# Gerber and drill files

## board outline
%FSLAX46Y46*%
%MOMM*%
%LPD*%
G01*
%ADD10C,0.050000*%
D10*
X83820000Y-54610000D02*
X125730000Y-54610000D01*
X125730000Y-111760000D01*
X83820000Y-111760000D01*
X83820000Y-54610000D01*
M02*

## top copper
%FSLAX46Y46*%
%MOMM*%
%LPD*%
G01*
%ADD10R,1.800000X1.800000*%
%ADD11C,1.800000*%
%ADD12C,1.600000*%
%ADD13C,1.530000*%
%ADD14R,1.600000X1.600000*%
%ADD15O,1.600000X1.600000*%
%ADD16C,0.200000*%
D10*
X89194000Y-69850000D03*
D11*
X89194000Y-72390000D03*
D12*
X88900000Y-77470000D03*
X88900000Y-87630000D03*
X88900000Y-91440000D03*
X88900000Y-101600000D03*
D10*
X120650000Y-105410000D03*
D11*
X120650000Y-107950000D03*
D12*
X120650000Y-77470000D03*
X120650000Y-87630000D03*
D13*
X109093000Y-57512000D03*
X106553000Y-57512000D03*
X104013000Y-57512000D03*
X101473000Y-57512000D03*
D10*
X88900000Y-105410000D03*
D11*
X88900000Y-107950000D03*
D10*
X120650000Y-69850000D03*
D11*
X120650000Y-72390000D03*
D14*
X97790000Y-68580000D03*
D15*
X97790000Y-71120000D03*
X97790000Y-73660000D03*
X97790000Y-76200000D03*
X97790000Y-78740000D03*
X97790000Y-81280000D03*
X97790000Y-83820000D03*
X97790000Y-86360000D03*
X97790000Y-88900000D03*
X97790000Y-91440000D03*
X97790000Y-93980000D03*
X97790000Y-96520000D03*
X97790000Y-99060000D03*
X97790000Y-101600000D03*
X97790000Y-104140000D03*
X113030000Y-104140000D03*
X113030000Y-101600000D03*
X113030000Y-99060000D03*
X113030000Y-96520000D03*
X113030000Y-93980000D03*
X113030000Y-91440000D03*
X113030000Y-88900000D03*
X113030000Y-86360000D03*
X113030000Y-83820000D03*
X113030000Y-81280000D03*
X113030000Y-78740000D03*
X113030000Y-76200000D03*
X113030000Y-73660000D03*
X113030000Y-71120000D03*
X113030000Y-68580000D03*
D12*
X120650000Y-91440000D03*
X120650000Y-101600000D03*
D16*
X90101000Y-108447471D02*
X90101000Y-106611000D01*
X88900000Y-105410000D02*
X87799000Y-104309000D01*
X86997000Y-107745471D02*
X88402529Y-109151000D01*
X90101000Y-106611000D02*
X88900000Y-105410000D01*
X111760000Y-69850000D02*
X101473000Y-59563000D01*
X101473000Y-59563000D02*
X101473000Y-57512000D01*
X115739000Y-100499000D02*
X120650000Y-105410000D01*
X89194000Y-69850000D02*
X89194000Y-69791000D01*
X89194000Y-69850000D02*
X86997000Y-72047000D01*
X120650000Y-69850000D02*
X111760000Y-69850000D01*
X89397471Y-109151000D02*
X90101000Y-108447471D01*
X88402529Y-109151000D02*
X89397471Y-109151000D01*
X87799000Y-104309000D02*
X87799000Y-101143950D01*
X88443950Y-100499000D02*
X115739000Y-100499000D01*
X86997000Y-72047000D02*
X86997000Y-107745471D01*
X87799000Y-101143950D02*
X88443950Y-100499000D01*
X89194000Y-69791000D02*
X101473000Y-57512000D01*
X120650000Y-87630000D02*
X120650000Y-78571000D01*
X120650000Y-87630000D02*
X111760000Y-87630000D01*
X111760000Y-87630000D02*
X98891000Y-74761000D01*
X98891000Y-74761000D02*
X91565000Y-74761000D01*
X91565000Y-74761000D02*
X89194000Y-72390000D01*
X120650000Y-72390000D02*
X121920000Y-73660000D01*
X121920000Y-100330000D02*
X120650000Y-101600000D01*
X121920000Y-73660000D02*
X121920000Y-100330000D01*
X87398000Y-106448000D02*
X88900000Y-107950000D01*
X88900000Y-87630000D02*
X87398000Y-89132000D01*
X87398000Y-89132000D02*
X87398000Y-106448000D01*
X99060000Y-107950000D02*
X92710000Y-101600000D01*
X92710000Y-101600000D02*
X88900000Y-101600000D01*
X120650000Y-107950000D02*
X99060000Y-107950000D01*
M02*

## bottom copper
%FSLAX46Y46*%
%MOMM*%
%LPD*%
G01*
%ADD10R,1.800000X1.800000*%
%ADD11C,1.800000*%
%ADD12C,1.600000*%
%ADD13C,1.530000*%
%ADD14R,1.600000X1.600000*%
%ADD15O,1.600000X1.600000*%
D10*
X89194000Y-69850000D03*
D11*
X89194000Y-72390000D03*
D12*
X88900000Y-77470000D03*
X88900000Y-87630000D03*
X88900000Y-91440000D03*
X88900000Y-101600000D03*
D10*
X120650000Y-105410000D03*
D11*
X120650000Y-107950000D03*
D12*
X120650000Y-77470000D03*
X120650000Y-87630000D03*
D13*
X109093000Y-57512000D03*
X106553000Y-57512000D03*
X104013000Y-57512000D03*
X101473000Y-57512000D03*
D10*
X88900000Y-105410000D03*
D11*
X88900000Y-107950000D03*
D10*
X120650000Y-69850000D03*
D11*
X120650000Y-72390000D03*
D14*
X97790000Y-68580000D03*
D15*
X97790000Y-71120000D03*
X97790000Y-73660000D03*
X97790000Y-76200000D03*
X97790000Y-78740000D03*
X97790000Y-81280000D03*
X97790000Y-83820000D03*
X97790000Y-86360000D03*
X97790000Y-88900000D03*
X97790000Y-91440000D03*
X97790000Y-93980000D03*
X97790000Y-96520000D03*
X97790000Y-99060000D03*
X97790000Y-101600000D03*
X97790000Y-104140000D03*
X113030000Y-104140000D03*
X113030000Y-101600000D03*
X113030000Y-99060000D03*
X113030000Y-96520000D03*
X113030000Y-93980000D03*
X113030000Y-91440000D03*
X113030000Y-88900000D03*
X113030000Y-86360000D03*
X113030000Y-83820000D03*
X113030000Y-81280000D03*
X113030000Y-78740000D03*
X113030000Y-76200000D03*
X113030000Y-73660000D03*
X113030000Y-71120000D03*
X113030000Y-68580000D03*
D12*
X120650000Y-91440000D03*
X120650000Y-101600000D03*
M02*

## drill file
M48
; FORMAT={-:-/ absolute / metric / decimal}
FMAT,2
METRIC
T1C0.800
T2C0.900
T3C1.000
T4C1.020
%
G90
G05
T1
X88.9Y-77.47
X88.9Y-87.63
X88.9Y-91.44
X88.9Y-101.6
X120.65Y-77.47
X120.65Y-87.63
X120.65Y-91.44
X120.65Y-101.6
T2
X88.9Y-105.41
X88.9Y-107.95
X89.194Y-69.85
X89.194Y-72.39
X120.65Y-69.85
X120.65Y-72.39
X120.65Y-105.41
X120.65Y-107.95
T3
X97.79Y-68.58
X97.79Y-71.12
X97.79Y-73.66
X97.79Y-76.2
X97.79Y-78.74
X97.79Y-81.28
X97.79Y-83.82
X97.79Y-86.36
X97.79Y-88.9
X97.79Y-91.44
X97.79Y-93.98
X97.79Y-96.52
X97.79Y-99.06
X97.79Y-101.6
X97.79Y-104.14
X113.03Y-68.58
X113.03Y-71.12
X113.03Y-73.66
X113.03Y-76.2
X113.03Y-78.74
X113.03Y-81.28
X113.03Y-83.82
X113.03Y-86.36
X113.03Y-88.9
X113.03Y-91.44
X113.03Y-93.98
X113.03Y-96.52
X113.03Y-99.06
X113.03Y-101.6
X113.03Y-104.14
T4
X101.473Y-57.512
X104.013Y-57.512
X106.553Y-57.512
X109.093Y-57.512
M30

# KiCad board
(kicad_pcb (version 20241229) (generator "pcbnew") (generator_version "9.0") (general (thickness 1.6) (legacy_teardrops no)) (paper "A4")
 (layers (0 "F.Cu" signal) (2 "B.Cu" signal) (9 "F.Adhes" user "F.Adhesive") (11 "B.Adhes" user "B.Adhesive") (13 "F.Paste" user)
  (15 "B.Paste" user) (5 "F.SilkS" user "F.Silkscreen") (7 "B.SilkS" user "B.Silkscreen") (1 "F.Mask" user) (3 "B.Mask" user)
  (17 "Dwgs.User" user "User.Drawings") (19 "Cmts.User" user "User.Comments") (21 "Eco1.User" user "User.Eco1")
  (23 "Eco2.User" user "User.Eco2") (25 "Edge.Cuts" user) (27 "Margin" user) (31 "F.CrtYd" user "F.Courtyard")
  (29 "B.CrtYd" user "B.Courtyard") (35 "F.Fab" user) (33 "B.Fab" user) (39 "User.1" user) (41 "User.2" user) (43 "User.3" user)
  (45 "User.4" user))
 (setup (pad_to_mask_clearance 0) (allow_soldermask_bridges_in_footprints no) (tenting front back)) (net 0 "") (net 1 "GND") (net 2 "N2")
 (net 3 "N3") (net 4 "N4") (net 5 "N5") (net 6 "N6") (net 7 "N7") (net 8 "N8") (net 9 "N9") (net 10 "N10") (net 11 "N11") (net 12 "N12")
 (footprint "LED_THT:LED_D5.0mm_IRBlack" (layer "F.Cu") (at 89.194 69.85 -90)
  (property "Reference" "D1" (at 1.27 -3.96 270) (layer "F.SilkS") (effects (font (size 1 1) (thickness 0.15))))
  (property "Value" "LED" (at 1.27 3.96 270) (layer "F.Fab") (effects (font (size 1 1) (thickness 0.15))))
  (pad "1" thru_hole rect (at 0 0 270) (size 1.8 1.8) (drill 0.9) (layers "*.Cu" "*.Mask") (remove_unused_layers no) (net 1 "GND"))
  (pad "2" thru_hole circle (at 2.54 0 270) (size 1.8 1.8) (drill 0.9) (layers "*.Cu" "*.Mask") (remove_unused_layers no) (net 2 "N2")))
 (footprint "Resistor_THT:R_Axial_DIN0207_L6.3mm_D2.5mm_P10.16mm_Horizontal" (layer "F.Cu") (at 88.9 77.47 -90)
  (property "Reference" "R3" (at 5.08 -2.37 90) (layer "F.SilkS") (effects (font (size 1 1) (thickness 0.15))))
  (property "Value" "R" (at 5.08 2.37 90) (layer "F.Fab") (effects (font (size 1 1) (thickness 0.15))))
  (pad "1" thru_hole circle (at 0 0 270) (size 1.6 1.6) (drill 0.8) (layers "*.Cu" "*.Mask") (remove_unused_layers no) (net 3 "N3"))
  (pad "2" thru_hole circle (at 10.16 0 270) (size 1.6 1.6) (drill 0.8) (layers "*.Cu" "*.Mask") (remove_unused_layers no) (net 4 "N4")))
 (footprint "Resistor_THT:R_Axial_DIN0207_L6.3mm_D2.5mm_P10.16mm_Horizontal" (layer "F.Cu") (at 88.9 91.44 -90)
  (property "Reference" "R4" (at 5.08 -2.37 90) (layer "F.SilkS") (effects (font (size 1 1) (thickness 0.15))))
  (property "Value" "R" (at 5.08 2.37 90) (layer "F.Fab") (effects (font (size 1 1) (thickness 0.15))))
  (pad "1" thru_hole circle (at 0 0 270) (size 1.6 1.6) (drill 0.8) (layers "*.Cu" "*.Mask") (remove_unused_layers no) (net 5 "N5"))
  (pad "2" thru_hole circle (at 10.16 0 270) (size 1.6 1.6) (drill 0.8) (layers "*.Cu" "*.Mask") (remove_unused_layers no) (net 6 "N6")))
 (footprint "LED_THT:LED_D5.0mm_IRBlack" (layer "F.Cu") (at 120.65 105.41 -90)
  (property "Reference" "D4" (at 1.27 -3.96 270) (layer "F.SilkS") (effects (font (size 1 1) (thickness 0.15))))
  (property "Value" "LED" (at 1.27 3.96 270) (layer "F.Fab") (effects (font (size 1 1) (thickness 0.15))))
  (pad "1" thru_hole rect (at 0 0 270) (size 1.8 1.8) (drill 0.9) (layers "*.Cu" "*.Mask") (remove_unused_layers no) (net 1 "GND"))
  (pad "2" thru_hole circle (at 2.54 0 270) (size 1.8 1.8) (drill 0.9) (layers "*.Cu" "*.Mask") (remove_unused_layers no) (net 6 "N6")))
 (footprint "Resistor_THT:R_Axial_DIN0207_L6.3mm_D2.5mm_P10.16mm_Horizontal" (layer "F.Cu") (at 120.65 77.47 -90)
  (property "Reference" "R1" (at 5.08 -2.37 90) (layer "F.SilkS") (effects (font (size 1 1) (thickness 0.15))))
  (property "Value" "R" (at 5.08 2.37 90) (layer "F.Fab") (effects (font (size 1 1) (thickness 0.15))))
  (pad "1" thru_hole circle (at 0 0 270) (size 1.6 1.6) (drill 0.8) (layers "*.Cu" "*.Mask") (remove_unused_layers no) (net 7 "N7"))
  (pad "2" thru_hole circle (at 10.16 0 270) (size 1.6 1.6) (drill 0.8) (layers "*.Cu" "*.Mask") (remove_unused_layers no) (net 2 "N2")))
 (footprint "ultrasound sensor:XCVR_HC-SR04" (layer "F.Cu") (at 105.283 57.512 180)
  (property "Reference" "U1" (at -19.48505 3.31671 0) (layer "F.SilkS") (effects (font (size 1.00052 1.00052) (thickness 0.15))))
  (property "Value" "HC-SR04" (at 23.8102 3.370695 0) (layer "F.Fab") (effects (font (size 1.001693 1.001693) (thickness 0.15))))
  (pad "1" thru_hole circle (at -3.81 0 180) (size 1.53 1.53) (drill 1.02) (layers "*.Cu" "*.Mask") (remove_unused_layers no) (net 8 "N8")
   (solder_mask_margin 0.102))
  (pad "2" thru_hole circle (at -1.27 0 180) (size 1.53 1.53) (drill 1.02) (layers "*.Cu" "*.Mask") (remove_unused_layers no) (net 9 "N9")
   (solder_mask_margin 0.102))
  (pad "3" thru_hole circle (at 1.27 0 180) (size 1.53 1.53) (drill 1.02) (layers "*.Cu" "*.Mask") (remove_unused_layers no) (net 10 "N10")
   (solder_mask_margin 0.102))
  (pad "4" thru_hole circle (at 3.81 0 180) (size 1.53 1.53) (drill 1.02) (layers "*.Cu" "*.Mask") (remove_unused_layers no) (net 1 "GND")
   (solder_mask_margin 0.102)))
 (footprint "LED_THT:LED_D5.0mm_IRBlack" (layer "F.Cu") (at 88.9 105.41 -90)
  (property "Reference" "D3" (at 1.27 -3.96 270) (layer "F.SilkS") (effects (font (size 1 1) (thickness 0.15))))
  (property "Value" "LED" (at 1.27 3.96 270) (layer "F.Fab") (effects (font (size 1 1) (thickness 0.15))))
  (pad "1" thru_hole rect (at 0 0 270) (size 1.8 1.8) (drill 0.9) (layers "*.Cu" "*.Mask") (remove_unused_layers no) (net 1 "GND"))
  (pad "2" thru_hole circle (at 2.54 0 270) (size 1.8 1.8) (drill 0.9) (layers "*.Cu" "*.Mask") (remove_unused_layers no) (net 4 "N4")))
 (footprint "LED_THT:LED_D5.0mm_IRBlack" (layer "F.Cu") (at 120.65 69.85 -90)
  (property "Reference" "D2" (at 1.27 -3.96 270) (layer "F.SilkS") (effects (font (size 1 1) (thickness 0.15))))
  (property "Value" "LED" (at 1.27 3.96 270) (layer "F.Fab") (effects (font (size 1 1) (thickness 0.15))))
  (pad "1" thru_hole rect (at 0 0 270) (size 1.8 1.8) (drill 0.9) (layers "*.Cu" "*.Mask") (remove_unused_layers no) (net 1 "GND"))
  (pad "2" thru_hole circle (at 2.54 0 270) (size 1.8 1.8) (drill 0.9) (layers "*.Cu" "*.Mask") (remove_unused_layers no) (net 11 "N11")))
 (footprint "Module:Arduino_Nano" (layer "F.Cu") (at 97.79 68.58)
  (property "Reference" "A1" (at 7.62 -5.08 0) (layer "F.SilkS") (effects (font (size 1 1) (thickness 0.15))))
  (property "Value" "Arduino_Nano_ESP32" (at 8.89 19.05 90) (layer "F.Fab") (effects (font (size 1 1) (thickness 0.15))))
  (pad "1" thru_hole rect (at 0 0) (size 1.6 1.6) (drill 1) (layers "*.Cu" "*.Mask") (remove_unused_layers no))
  (pad "2" thru_hole oval (at 0 2.54) (size 1.6 1.6) (drill 1) (layers "*.Cu" "*.Mask") (remove_unused_layers no))
  (pad "3" thru_hole oval (at 0 5.08) (size 1.6 1.6) (drill 1) (layers "*.Cu" "*.Mask") (remove_unused_layers no))
  (pad "4" thru_hole oval (at 0 7.62) (size 1.6 1.6) (drill 1) (layers "*.Cu" "*.Mask") (remove_unused_layers no))
  (pad "5" thru_hole oval (at 0 10.16) (size 1.6 1.6) (drill 1) (layers "*.Cu" "*.Mask") (remove_unused_layers no))
  (pad "6" thru_hole oval (at 0 12.7) (size 1.6 1.6) (drill 1) (layers "*.Cu" "*.Mask") (remove_unused_layers no))
  (pad "7" thru_hole oval (at 0 15.24) (size 1.6 1.6) (drill 1) (layers "*.Cu" "*.Mask") (remove_unused_layers no))
  (pad "8" thru_hole oval (at 0 17.78) (size 1.6 1.6) (drill 1) (layers "*.Cu" "*.Mask") (remove_unused_layers no))
  (pad "9" thru_hole oval (at 0 20.32) (size 1.6 1.6) (drill 1) (layers "*.Cu" "*.Mask") (remove_unused_layers no))
  (pad "10" thru_hole oval (at 0 22.86) (size 1.6 1.6) (drill 1) (layers "*.Cu" "*.Mask") (remove_unused_layers no))
  (pad "11" thru_hole oval (at 0 25.4) (size 1.6 1.6) (drill 1) (layers "*.Cu" "*.Mask") (remove_unused_layers no))
  (pad "12" thru_hole oval (at 0 27.94) (size 1.6 1.6) (drill 1) (layers "*.Cu" "*.Mask") (remove_unused_layers no))
  (pad "13" thru_hole oval (at 0 30.48) (size 1.6 1.6) (drill 1) (layers "*.Cu" "*.Mask") (remove_unused_layers no))
  (pad "14" thru_hole oval (at 0 33.02) (size 1.6 1.6) (drill 1) (layers "*.Cu" "*.Mask") (remove_unused_layers no))
  (pad "15" thru_hole oval (at 0 35.56) (size 1.6 1.6) (drill 1) (layers "*.Cu" "*.Mask") (remove_unused_layers no))
  (pad "16" thru_hole oval (at 15.24 35.56) (size 1.6 1.6) (drill 1) (layers "*.Cu" "*.Mask") (remove_unused_layers no))
  (pad "17" thru_hole oval (at 15.24 33.02) (size 1.6 1.6) (drill 1) (layers "*.Cu" "*.Mask") (remove_unused_layers no))
  (pad "18" thru_hole oval (at 15.24 30.48) (size 1.6 1.6) (drill 1) (layers "*.Cu" "*.Mask") (remove_unused_layers no))
  (pad "19" thru_hole oval (at 15.24 27.94) (size 1.6 1.6) (drill 1) (layers "*.Cu" "*.Mask") (remove_unused_layers no))
  (pad "20" thru_hole oval (at 15.24 25.4) (size 1.6 1.6) (drill 1) (layers "*.Cu" "*.Mask") (remove_unused_layers no))
  (pad "21" thru_hole oval (at 15.24 22.86) (size 1.6 1.6) (drill 1) (layers "*.Cu" "*.Mask") (remove_unused_layers no))
  (pad "22" thru_hole oval (at 15.24 20.32) (size 1.6 1.6) (drill 1) (layers "*.Cu" "*.Mask") (remove_unused_layers no))
  (pad "23" thru_hole oval (at 15.24 17.78) (size 1.6 1.6) (drill 1) (layers "*.Cu" "*.Mask") (remove_unused_layers no))
  (pad "24" thru_hole oval (at 15.24 15.24) (size 1.6 1.6) (drill 1) (layers "*.Cu" "*.Mask") (remove_unused_layers no))
  (pad "25" thru_hole oval (at 15.24 12.7) (size 1.6 1.6) (drill 1) (layers "*.Cu" "*.Mask") (remove_unused_layers no))
  (pad "26" thru_hole oval (at 15.24 10.16) (size 1.6 1.6) (drill 1) (layers "*.Cu" "*.Mask") (remove_unused_layers no))
  (pad "27" thru_hole oval (at 15.24 7.62) (size 1.6 1.6) (drill 1) (layers "*.Cu" "*.Mask") (remove_unused_layers no))
  (pad "28" thru_hole oval (at 15.24 5.08) (size 1.6 1.6) (drill 1) (layers "*.Cu" "*.Mask") (remove_unused_layers no))
  (pad "29" thru_hole oval (at 15.24 2.54) (size 1.6 1.6) (drill 1) (layers "*.Cu" "*.Mask") (remove_unused_layers no))
  (pad "30" thru_hole oval (at 15.24 0) (size 1.6 1.6) (drill 1) (layers "*.Cu" "*.Mask") (remove_unused_layers no)))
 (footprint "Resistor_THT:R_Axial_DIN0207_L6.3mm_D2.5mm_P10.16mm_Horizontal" (layer "F.Cu") (at 120.65 91.44 -90)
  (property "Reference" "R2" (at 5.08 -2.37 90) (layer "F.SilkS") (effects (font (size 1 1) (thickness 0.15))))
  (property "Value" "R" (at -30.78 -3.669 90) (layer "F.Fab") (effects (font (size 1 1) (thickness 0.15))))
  (pad "1" thru_hole circle (at 0 0 270) (size 1.6 1.6) (drill 0.8) (layers "*.Cu" "*.Mask") (remove_unused_layers no) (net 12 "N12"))
  (pad "2" thru_hole circle (at 10.16 0 270) (size 1.6 1.6) (drill 0.8) (layers "*.Cu" "*.Mask") (remove_unused_layers no) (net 11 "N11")))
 (gr_rect (start 83.82 54.61) (end 125.73 111.76) (stroke (width 0.05) (type default)) (fill no) (layer "Edge.Cuts"))
 (segment (start 90.101 108.447471) (end 90.101 106.611) (width 0.2) (layer "F.Cu") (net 1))
 (segment (start 88.9 105.41) (end 87.799 104.309) (width 0.2) (layer "F.Cu") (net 1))
 (segment (start 86.997 107.745471) (end 88.402529 109.151) (width 0.2) (layer "F.Cu") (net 1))
 (segment (start 90.101 106.611) (end 88.9 105.41) (width 0.2) (layer "F.Cu") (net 1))
 (segment (start 111.76 69.85) (end 101.473 59.563) (width 0.2) (layer "F.Cu") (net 1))
 (segment (start 101.473 59.563) (end 101.473 57.512) (width 0.2) (layer "F.Cu") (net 1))
 (segment (start 115.739 100.499) (end 120.65 105.41) (width 0.2) (layer "F.Cu") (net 1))
 (segment (start 89.194 69.85) (end 89.194 69.791) (width 0.2) (layer "F.Cu") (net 1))
 (segment (start 89.194 69.85) (end 86.997 72.047) (width 0.2) (layer "F.Cu") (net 1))
 (segment (start 120.65 69.85) (end 111.76 69.85) (width 0.2) (layer "F.Cu") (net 1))
 (segment (start 89.397471 109.151) (end 90.101 108.447471) (width 0.2) (layer "F.Cu") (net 1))
 (segment (start 88.402529 109.151) (end 89.397471 109.151) (width 0.2) (layer "F.Cu") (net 1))
 (segment (start 87.799 104.309) (end 87.799 101.14395) (width 0.2) (layer "F.Cu") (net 1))
 (segment (start 88.44395 100.499) (end 115.739 100.499) (width 0.2) (layer "F.Cu") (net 1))
 (segment (start 86.997 72.047) (end 86.997 107.745471) (width 0.2) (layer "F.Cu") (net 1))
 (segment (start 87.799 101.14395) (end 88.44395 100.499) (width 0.2) (layer "F.Cu") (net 1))
 (segment (start 89.194 69.791) (end 101.473 57.512) (width 0.2) (layer "F.Cu") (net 1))
 (segment (start 120.65 87.63) (end 120.65 78.571) (width 0.2) (layer "F.Cu") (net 2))
 (segment (start 120.65 87.63) (end 111.76 87.63) (width 0.2) (layer "F.Cu") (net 2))
 (segment (start 111.76 87.63) (end 98.891 74.761) (width 0.2) (layer "F.Cu") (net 2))
 (segment (start 98.891 74.761) (end 91.565 74.761) (width 0.2) (layer "F.Cu") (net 2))
 (segment (start 91.565 74.761) (end 89.194 72.39) (width 0.2) (layer "F.Cu") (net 2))
 (segment (start 120.65 72.39) (end 121.92 73.66) (width 0.2) (layer "F.Cu") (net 11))
 (segment (start 121.92 100.33) (end 120.65 101.6) (width 0.2) (layer "F.Cu") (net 11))
 (segment (start 121.92 73.66) (end 121.92 100.33) (width 0.2) (layer "F.Cu") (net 11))
 (segment (start 87.398 106.448) (end 88.9 107.95) (width 0.2) (layer "F.Cu") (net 4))
 (segment (start 88.9 87.63) (end 87.398 89.132) (width 0.2) (layer "F.Cu") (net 4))
 (segment (start 87.398 89.132) (end 87.398 106.448) (width 0.2) (layer "F.Cu") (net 4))
 (segment (start 99.06 107.95) (end 92.71 101.6) (width 0.2) (layer "F.Cu") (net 6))
 (segment (start 92.71 101.6) (end 88.9 101.6) (width 0.2) (layer "F.Cu") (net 6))
 (segment (start 120.65 107.95) (end 99.06 107.95) (width 0.2) (layer "F.Cu") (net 6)))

